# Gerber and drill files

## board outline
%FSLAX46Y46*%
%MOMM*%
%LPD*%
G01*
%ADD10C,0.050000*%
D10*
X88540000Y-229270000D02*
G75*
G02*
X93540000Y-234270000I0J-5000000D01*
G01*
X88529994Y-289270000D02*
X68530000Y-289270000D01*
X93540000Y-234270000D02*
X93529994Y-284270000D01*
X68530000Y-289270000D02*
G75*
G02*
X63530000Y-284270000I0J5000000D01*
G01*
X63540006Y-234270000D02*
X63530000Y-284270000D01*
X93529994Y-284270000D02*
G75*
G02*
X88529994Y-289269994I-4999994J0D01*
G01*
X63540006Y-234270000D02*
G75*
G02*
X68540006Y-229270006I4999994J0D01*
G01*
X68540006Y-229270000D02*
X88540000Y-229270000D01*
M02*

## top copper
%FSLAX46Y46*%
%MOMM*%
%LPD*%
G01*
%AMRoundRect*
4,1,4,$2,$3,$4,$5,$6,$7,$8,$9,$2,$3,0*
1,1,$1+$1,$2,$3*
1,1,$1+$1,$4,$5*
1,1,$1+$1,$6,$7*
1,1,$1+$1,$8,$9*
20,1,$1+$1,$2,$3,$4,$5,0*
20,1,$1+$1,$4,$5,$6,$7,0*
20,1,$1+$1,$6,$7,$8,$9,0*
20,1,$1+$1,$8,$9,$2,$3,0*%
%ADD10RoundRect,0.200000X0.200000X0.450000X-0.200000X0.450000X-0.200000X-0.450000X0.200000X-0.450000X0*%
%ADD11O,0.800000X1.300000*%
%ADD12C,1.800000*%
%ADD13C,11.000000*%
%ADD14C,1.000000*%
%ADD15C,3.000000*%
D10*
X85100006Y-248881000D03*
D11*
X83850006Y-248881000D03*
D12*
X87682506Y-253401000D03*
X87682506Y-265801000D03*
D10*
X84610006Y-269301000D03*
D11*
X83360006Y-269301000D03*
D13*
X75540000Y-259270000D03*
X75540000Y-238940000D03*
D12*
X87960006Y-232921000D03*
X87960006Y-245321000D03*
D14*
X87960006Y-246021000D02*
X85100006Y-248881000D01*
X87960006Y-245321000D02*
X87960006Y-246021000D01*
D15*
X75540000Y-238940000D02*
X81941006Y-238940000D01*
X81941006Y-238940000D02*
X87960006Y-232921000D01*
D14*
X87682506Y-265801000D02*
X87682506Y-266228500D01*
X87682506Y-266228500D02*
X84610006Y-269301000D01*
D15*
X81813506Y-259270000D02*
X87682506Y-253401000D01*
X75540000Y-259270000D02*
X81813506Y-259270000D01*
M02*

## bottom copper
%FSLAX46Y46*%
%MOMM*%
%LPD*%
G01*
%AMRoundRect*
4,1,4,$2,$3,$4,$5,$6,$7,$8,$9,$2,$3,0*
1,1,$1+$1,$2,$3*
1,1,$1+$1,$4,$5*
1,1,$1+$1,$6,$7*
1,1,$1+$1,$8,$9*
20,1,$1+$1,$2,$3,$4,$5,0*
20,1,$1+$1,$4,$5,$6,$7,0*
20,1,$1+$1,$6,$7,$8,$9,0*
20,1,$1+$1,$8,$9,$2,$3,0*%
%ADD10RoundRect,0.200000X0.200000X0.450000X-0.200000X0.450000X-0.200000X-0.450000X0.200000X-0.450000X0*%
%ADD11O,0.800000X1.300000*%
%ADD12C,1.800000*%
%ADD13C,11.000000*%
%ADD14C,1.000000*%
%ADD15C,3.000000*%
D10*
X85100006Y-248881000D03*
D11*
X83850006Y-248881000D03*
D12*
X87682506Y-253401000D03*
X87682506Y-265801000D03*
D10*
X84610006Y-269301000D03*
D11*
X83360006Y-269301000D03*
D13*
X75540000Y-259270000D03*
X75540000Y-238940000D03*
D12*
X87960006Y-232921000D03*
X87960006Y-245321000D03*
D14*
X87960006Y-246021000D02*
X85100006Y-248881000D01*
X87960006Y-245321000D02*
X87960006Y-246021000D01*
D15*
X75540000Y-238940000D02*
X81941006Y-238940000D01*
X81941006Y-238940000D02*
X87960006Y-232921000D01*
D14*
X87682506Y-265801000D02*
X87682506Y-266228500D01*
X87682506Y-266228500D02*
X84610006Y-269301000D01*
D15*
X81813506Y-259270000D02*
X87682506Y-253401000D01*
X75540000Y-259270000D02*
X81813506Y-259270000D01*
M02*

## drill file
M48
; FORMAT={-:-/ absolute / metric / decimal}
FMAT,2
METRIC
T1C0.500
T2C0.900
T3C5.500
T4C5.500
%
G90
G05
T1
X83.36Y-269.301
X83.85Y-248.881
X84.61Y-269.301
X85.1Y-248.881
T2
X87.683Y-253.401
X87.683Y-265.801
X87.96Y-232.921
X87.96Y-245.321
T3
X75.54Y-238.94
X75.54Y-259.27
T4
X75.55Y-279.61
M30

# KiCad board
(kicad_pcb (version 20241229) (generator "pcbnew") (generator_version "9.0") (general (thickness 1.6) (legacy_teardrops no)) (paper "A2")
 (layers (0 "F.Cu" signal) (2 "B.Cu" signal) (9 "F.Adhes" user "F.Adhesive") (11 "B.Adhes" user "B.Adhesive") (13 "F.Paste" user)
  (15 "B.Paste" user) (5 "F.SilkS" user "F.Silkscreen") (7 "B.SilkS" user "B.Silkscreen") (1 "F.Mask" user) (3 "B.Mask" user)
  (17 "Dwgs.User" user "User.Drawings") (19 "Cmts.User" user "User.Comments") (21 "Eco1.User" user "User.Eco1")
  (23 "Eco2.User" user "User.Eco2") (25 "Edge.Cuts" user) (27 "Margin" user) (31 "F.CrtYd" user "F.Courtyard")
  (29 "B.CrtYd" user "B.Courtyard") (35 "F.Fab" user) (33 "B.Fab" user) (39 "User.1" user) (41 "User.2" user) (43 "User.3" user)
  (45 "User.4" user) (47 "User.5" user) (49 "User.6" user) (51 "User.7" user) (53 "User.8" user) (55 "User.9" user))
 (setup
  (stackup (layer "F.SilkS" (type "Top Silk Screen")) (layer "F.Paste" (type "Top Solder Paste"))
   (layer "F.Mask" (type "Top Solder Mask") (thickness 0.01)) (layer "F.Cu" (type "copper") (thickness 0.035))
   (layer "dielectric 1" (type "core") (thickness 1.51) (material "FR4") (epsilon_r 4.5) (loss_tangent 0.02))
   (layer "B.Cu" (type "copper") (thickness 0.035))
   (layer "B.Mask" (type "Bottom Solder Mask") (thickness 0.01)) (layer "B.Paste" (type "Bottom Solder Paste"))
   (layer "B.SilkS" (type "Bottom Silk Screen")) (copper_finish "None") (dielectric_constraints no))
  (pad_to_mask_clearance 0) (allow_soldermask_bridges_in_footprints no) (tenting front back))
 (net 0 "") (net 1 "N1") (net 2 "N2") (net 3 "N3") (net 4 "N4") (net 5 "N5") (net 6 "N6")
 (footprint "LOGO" (layer "F.Cu") (at 89.18 283.61 90)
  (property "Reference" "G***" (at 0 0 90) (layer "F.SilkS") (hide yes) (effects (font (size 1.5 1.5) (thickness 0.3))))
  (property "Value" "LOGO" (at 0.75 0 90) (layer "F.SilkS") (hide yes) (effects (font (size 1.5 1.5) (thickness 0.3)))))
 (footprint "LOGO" (layer "F.Cu") (at 89.86 273.92 90)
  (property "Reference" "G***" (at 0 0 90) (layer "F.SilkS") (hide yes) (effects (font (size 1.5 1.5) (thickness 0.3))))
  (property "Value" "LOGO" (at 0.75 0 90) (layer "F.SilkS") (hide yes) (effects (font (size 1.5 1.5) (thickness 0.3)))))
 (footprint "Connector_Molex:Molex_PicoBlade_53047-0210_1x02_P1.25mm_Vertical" (layer "F.Cu") (at 85.100006 248.881 180)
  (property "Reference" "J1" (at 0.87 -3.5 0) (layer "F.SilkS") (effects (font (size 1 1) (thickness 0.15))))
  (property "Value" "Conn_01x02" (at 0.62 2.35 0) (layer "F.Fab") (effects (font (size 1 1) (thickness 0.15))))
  (pad "1" thru_hole roundrect (at 0 0 180) (size 0.8 1.3) (drill 0.5) (layers "*.Cu" "*.Mask") (remove_unused_layers no)
   (roundrect_rratio 0.25) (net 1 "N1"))
  (pad "2" thru_hole oval (at 1.25 0 180) (size 0.8 1.3) (drill 0.5) (layers "*.Cu" "*.Mask") (remove_unused_layers no) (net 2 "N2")))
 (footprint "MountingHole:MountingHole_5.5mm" (layer "F.Cu") (at 75.55 279.61)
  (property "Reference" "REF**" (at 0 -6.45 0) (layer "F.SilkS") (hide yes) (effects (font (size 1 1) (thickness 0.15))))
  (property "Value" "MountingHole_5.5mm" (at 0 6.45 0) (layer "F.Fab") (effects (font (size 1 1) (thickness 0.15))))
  (pad "" np_thru_hole circle (at 0 0) (size 5.5 5.5) (drill 5.5) (layers "*.Cu" "*.Mask")))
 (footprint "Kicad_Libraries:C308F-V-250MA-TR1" (layer "F.Cu") (at 94.282506 259.001 -90)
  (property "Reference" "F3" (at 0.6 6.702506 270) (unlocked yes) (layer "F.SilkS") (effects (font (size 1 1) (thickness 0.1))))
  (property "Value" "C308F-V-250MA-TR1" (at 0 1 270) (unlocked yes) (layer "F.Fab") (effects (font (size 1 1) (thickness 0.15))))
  (pad "1" thru_hole circle (at -5.6 6.6 270) (size 1.8 1.8) (drill 0.9) (layers "*.Cu" "*.Mask") (remove_unused_layers no) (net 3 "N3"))
  (pad "2" thru_hole circle (at 6.8 6.6 270) (size 1.8 1.8) (drill 0.9) (layers "*.Cu" "*.Mask") (remove_unused_layers no) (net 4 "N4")))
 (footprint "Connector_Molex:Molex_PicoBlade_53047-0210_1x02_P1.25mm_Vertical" (layer "F.Cu") (at 84.610006 269.301 180)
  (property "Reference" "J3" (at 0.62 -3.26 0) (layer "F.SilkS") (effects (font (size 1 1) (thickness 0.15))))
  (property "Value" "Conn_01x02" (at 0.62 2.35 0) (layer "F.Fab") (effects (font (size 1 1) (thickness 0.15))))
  (pad "1" thru_hole roundrect (at 0 0 180) (size 0.8 1.3) (drill 0.5) (layers "*.Cu" "*.Mask") (remove_unused_layers no)
   (roundrect_rratio 0.25) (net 4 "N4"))
  (pad "2" thru_hole oval (at 1.25 0 180) (size 0.8 1.3) (drill 0.5) (layers "*.Cu" "*.Mask") (remove_unused_layers no) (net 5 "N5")))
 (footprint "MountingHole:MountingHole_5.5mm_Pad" (layer "F.Cu") (at 75.54 259.27)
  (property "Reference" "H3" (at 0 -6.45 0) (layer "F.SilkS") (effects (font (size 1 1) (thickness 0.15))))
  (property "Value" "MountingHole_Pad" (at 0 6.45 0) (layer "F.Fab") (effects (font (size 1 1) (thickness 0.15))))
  (pad "1" thru_hole circle (at 0 0) (size 11 11) (drill 5.5) (layers "*.Cu" "*.Mask") (remove_unused_layers no) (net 3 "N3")
   (zone_connect 2)))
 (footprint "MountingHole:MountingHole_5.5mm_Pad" (layer "F.Cu") (at 75.54 238.94)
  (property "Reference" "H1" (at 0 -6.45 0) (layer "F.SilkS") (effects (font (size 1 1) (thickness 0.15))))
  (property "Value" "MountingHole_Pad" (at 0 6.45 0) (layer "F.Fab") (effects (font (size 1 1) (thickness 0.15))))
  (pad "1" thru_hole circle (at 0 0) (size 11 11) (drill 5.5) (layers "*.Cu" "*.Mask") (remove_unused_layers no) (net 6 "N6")
   (zone_connect 2)))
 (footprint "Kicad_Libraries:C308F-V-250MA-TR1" (layer "F.Cu") (at 94.560006 238.521 -90)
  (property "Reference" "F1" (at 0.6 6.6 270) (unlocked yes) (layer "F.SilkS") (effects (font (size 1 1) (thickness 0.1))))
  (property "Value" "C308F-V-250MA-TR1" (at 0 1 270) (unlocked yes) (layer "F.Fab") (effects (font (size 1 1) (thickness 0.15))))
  (pad "1" thru_hole circle (at -5.6 6.6 270) (size 1.8 1.8) (drill 0.9) (layers "*.Cu" "*.Mask") (remove_unused_layers no) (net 6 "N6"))
  (pad "2" thru_hole circle (at 6.8 6.6 270) (size 1.8 1.8) (drill 0.9) (layers "*.Cu" "*.Mask") (remove_unused_layers no) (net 1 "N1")))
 (gr_arc (start 88.54 229.27) (mid 92.075534 230.734466) (end 93.54 234.27) (stroke (width 0.05) (type default)) (layer "Edge.Cuts"))
 (gr_line (start 88.529994 289.27) (end 68.53 289.27) (stroke (width 0.05) (type default)) (layer "Edge.Cuts"))
 (gr_line (start 93.54 234.27) (end 93.529994 284.27) (stroke (width 0.05) (type default)) (layer "Edge.Cuts"))
 (gr_arc (start 68.53 289.27) (mid 64.994466 287.805534) (end 63.53 284.27) (stroke (width 0.05) (type default)) (layer "Edge.Cuts"))
 (gr_line (start 63.540006 234.27) (end 63.53 284.27) (stroke (width 0.05) (type default)) (layer "Edge.Cuts"))
 (gr_arc (start 93.529994 284.27) (mid 92.065528 287.805534) (end 88.529994 289.27) (stroke (width 0.05) (type default)) (layer "Edge.Cuts"))
 (gr_arc (start 63.540006 234.27) (mid 65.004472 230.734466) (end 68.540006 229.27) (stroke (width 0.05) (type default)) (layer "Edge.Cuts"))
 (gr_line (start 68.540006 229.27) (end 88.54 229.27) (stroke (width 0.05) (type default)) (layer "Edge.Cuts"))
 (segment (start 87.960006 246.021) (end 85.100006 248.881) (width 1) (layer "F.Cu") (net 1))
 (segment (start 87.960006 245.321) (end 87.960006 246.021) (width 1) (layer "F.Cu") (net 1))
 (segment (start 87.960006 246.021) (end 85.100006 248.881) (width 1) (layer "B.Cu") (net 1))
 (segment (start 87.960006 245.321) (end 87.960006 246.021) (width 1) (layer "B.Cu") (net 1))
 (segment (start 75.54 238.94) (end 81.941006 238.94) (width 3) (layer "F.Cu") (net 6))
 (segment (start 81.941006 238.94) (end 87.960006 232.921) (width 3) (layer "F.Cu") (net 6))
 (segment (start 75.54 238.94) (end 81.941006 238.94) (width 3) (layer "B.Cu") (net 6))
 (segment (start 81.941006 238.94) (end 87.960006 232.921) (width 3) (layer "B.Cu") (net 6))
 (segment (start 87.682506 265.801) (end 87.682506 266.2285) (width 1) (layer "F.Cu") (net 4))
 (segment (start 87.682506 266.2285) (end 84.610006 269.301) (width 1) (layer "F.Cu") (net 4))
 (segment (start 87.682506 265.801) (end 87.682506 266.2285) (width 1) (layer "B.Cu") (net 4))
 (segment (start 87.682506 266.2285) (end 84.610006 269.301) (width 1) (layer "B.Cu") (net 4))
 (segment (start 81.813506 259.27) (end 87.682506 253.401) (width 3) (layer "F.Cu") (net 3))
 (segment (start 75.54 259.27) (end 81.813506 259.27) (width 3) (layer "F.Cu") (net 3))
 (segment (start 81.813506 259.27) (end 87.682506 253.401) (width 3) (layer "B.Cu") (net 3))
 (segment (start 75.54 259.27) (end 81.813506 259.27) (width 3) (layer "B.Cu") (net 3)))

